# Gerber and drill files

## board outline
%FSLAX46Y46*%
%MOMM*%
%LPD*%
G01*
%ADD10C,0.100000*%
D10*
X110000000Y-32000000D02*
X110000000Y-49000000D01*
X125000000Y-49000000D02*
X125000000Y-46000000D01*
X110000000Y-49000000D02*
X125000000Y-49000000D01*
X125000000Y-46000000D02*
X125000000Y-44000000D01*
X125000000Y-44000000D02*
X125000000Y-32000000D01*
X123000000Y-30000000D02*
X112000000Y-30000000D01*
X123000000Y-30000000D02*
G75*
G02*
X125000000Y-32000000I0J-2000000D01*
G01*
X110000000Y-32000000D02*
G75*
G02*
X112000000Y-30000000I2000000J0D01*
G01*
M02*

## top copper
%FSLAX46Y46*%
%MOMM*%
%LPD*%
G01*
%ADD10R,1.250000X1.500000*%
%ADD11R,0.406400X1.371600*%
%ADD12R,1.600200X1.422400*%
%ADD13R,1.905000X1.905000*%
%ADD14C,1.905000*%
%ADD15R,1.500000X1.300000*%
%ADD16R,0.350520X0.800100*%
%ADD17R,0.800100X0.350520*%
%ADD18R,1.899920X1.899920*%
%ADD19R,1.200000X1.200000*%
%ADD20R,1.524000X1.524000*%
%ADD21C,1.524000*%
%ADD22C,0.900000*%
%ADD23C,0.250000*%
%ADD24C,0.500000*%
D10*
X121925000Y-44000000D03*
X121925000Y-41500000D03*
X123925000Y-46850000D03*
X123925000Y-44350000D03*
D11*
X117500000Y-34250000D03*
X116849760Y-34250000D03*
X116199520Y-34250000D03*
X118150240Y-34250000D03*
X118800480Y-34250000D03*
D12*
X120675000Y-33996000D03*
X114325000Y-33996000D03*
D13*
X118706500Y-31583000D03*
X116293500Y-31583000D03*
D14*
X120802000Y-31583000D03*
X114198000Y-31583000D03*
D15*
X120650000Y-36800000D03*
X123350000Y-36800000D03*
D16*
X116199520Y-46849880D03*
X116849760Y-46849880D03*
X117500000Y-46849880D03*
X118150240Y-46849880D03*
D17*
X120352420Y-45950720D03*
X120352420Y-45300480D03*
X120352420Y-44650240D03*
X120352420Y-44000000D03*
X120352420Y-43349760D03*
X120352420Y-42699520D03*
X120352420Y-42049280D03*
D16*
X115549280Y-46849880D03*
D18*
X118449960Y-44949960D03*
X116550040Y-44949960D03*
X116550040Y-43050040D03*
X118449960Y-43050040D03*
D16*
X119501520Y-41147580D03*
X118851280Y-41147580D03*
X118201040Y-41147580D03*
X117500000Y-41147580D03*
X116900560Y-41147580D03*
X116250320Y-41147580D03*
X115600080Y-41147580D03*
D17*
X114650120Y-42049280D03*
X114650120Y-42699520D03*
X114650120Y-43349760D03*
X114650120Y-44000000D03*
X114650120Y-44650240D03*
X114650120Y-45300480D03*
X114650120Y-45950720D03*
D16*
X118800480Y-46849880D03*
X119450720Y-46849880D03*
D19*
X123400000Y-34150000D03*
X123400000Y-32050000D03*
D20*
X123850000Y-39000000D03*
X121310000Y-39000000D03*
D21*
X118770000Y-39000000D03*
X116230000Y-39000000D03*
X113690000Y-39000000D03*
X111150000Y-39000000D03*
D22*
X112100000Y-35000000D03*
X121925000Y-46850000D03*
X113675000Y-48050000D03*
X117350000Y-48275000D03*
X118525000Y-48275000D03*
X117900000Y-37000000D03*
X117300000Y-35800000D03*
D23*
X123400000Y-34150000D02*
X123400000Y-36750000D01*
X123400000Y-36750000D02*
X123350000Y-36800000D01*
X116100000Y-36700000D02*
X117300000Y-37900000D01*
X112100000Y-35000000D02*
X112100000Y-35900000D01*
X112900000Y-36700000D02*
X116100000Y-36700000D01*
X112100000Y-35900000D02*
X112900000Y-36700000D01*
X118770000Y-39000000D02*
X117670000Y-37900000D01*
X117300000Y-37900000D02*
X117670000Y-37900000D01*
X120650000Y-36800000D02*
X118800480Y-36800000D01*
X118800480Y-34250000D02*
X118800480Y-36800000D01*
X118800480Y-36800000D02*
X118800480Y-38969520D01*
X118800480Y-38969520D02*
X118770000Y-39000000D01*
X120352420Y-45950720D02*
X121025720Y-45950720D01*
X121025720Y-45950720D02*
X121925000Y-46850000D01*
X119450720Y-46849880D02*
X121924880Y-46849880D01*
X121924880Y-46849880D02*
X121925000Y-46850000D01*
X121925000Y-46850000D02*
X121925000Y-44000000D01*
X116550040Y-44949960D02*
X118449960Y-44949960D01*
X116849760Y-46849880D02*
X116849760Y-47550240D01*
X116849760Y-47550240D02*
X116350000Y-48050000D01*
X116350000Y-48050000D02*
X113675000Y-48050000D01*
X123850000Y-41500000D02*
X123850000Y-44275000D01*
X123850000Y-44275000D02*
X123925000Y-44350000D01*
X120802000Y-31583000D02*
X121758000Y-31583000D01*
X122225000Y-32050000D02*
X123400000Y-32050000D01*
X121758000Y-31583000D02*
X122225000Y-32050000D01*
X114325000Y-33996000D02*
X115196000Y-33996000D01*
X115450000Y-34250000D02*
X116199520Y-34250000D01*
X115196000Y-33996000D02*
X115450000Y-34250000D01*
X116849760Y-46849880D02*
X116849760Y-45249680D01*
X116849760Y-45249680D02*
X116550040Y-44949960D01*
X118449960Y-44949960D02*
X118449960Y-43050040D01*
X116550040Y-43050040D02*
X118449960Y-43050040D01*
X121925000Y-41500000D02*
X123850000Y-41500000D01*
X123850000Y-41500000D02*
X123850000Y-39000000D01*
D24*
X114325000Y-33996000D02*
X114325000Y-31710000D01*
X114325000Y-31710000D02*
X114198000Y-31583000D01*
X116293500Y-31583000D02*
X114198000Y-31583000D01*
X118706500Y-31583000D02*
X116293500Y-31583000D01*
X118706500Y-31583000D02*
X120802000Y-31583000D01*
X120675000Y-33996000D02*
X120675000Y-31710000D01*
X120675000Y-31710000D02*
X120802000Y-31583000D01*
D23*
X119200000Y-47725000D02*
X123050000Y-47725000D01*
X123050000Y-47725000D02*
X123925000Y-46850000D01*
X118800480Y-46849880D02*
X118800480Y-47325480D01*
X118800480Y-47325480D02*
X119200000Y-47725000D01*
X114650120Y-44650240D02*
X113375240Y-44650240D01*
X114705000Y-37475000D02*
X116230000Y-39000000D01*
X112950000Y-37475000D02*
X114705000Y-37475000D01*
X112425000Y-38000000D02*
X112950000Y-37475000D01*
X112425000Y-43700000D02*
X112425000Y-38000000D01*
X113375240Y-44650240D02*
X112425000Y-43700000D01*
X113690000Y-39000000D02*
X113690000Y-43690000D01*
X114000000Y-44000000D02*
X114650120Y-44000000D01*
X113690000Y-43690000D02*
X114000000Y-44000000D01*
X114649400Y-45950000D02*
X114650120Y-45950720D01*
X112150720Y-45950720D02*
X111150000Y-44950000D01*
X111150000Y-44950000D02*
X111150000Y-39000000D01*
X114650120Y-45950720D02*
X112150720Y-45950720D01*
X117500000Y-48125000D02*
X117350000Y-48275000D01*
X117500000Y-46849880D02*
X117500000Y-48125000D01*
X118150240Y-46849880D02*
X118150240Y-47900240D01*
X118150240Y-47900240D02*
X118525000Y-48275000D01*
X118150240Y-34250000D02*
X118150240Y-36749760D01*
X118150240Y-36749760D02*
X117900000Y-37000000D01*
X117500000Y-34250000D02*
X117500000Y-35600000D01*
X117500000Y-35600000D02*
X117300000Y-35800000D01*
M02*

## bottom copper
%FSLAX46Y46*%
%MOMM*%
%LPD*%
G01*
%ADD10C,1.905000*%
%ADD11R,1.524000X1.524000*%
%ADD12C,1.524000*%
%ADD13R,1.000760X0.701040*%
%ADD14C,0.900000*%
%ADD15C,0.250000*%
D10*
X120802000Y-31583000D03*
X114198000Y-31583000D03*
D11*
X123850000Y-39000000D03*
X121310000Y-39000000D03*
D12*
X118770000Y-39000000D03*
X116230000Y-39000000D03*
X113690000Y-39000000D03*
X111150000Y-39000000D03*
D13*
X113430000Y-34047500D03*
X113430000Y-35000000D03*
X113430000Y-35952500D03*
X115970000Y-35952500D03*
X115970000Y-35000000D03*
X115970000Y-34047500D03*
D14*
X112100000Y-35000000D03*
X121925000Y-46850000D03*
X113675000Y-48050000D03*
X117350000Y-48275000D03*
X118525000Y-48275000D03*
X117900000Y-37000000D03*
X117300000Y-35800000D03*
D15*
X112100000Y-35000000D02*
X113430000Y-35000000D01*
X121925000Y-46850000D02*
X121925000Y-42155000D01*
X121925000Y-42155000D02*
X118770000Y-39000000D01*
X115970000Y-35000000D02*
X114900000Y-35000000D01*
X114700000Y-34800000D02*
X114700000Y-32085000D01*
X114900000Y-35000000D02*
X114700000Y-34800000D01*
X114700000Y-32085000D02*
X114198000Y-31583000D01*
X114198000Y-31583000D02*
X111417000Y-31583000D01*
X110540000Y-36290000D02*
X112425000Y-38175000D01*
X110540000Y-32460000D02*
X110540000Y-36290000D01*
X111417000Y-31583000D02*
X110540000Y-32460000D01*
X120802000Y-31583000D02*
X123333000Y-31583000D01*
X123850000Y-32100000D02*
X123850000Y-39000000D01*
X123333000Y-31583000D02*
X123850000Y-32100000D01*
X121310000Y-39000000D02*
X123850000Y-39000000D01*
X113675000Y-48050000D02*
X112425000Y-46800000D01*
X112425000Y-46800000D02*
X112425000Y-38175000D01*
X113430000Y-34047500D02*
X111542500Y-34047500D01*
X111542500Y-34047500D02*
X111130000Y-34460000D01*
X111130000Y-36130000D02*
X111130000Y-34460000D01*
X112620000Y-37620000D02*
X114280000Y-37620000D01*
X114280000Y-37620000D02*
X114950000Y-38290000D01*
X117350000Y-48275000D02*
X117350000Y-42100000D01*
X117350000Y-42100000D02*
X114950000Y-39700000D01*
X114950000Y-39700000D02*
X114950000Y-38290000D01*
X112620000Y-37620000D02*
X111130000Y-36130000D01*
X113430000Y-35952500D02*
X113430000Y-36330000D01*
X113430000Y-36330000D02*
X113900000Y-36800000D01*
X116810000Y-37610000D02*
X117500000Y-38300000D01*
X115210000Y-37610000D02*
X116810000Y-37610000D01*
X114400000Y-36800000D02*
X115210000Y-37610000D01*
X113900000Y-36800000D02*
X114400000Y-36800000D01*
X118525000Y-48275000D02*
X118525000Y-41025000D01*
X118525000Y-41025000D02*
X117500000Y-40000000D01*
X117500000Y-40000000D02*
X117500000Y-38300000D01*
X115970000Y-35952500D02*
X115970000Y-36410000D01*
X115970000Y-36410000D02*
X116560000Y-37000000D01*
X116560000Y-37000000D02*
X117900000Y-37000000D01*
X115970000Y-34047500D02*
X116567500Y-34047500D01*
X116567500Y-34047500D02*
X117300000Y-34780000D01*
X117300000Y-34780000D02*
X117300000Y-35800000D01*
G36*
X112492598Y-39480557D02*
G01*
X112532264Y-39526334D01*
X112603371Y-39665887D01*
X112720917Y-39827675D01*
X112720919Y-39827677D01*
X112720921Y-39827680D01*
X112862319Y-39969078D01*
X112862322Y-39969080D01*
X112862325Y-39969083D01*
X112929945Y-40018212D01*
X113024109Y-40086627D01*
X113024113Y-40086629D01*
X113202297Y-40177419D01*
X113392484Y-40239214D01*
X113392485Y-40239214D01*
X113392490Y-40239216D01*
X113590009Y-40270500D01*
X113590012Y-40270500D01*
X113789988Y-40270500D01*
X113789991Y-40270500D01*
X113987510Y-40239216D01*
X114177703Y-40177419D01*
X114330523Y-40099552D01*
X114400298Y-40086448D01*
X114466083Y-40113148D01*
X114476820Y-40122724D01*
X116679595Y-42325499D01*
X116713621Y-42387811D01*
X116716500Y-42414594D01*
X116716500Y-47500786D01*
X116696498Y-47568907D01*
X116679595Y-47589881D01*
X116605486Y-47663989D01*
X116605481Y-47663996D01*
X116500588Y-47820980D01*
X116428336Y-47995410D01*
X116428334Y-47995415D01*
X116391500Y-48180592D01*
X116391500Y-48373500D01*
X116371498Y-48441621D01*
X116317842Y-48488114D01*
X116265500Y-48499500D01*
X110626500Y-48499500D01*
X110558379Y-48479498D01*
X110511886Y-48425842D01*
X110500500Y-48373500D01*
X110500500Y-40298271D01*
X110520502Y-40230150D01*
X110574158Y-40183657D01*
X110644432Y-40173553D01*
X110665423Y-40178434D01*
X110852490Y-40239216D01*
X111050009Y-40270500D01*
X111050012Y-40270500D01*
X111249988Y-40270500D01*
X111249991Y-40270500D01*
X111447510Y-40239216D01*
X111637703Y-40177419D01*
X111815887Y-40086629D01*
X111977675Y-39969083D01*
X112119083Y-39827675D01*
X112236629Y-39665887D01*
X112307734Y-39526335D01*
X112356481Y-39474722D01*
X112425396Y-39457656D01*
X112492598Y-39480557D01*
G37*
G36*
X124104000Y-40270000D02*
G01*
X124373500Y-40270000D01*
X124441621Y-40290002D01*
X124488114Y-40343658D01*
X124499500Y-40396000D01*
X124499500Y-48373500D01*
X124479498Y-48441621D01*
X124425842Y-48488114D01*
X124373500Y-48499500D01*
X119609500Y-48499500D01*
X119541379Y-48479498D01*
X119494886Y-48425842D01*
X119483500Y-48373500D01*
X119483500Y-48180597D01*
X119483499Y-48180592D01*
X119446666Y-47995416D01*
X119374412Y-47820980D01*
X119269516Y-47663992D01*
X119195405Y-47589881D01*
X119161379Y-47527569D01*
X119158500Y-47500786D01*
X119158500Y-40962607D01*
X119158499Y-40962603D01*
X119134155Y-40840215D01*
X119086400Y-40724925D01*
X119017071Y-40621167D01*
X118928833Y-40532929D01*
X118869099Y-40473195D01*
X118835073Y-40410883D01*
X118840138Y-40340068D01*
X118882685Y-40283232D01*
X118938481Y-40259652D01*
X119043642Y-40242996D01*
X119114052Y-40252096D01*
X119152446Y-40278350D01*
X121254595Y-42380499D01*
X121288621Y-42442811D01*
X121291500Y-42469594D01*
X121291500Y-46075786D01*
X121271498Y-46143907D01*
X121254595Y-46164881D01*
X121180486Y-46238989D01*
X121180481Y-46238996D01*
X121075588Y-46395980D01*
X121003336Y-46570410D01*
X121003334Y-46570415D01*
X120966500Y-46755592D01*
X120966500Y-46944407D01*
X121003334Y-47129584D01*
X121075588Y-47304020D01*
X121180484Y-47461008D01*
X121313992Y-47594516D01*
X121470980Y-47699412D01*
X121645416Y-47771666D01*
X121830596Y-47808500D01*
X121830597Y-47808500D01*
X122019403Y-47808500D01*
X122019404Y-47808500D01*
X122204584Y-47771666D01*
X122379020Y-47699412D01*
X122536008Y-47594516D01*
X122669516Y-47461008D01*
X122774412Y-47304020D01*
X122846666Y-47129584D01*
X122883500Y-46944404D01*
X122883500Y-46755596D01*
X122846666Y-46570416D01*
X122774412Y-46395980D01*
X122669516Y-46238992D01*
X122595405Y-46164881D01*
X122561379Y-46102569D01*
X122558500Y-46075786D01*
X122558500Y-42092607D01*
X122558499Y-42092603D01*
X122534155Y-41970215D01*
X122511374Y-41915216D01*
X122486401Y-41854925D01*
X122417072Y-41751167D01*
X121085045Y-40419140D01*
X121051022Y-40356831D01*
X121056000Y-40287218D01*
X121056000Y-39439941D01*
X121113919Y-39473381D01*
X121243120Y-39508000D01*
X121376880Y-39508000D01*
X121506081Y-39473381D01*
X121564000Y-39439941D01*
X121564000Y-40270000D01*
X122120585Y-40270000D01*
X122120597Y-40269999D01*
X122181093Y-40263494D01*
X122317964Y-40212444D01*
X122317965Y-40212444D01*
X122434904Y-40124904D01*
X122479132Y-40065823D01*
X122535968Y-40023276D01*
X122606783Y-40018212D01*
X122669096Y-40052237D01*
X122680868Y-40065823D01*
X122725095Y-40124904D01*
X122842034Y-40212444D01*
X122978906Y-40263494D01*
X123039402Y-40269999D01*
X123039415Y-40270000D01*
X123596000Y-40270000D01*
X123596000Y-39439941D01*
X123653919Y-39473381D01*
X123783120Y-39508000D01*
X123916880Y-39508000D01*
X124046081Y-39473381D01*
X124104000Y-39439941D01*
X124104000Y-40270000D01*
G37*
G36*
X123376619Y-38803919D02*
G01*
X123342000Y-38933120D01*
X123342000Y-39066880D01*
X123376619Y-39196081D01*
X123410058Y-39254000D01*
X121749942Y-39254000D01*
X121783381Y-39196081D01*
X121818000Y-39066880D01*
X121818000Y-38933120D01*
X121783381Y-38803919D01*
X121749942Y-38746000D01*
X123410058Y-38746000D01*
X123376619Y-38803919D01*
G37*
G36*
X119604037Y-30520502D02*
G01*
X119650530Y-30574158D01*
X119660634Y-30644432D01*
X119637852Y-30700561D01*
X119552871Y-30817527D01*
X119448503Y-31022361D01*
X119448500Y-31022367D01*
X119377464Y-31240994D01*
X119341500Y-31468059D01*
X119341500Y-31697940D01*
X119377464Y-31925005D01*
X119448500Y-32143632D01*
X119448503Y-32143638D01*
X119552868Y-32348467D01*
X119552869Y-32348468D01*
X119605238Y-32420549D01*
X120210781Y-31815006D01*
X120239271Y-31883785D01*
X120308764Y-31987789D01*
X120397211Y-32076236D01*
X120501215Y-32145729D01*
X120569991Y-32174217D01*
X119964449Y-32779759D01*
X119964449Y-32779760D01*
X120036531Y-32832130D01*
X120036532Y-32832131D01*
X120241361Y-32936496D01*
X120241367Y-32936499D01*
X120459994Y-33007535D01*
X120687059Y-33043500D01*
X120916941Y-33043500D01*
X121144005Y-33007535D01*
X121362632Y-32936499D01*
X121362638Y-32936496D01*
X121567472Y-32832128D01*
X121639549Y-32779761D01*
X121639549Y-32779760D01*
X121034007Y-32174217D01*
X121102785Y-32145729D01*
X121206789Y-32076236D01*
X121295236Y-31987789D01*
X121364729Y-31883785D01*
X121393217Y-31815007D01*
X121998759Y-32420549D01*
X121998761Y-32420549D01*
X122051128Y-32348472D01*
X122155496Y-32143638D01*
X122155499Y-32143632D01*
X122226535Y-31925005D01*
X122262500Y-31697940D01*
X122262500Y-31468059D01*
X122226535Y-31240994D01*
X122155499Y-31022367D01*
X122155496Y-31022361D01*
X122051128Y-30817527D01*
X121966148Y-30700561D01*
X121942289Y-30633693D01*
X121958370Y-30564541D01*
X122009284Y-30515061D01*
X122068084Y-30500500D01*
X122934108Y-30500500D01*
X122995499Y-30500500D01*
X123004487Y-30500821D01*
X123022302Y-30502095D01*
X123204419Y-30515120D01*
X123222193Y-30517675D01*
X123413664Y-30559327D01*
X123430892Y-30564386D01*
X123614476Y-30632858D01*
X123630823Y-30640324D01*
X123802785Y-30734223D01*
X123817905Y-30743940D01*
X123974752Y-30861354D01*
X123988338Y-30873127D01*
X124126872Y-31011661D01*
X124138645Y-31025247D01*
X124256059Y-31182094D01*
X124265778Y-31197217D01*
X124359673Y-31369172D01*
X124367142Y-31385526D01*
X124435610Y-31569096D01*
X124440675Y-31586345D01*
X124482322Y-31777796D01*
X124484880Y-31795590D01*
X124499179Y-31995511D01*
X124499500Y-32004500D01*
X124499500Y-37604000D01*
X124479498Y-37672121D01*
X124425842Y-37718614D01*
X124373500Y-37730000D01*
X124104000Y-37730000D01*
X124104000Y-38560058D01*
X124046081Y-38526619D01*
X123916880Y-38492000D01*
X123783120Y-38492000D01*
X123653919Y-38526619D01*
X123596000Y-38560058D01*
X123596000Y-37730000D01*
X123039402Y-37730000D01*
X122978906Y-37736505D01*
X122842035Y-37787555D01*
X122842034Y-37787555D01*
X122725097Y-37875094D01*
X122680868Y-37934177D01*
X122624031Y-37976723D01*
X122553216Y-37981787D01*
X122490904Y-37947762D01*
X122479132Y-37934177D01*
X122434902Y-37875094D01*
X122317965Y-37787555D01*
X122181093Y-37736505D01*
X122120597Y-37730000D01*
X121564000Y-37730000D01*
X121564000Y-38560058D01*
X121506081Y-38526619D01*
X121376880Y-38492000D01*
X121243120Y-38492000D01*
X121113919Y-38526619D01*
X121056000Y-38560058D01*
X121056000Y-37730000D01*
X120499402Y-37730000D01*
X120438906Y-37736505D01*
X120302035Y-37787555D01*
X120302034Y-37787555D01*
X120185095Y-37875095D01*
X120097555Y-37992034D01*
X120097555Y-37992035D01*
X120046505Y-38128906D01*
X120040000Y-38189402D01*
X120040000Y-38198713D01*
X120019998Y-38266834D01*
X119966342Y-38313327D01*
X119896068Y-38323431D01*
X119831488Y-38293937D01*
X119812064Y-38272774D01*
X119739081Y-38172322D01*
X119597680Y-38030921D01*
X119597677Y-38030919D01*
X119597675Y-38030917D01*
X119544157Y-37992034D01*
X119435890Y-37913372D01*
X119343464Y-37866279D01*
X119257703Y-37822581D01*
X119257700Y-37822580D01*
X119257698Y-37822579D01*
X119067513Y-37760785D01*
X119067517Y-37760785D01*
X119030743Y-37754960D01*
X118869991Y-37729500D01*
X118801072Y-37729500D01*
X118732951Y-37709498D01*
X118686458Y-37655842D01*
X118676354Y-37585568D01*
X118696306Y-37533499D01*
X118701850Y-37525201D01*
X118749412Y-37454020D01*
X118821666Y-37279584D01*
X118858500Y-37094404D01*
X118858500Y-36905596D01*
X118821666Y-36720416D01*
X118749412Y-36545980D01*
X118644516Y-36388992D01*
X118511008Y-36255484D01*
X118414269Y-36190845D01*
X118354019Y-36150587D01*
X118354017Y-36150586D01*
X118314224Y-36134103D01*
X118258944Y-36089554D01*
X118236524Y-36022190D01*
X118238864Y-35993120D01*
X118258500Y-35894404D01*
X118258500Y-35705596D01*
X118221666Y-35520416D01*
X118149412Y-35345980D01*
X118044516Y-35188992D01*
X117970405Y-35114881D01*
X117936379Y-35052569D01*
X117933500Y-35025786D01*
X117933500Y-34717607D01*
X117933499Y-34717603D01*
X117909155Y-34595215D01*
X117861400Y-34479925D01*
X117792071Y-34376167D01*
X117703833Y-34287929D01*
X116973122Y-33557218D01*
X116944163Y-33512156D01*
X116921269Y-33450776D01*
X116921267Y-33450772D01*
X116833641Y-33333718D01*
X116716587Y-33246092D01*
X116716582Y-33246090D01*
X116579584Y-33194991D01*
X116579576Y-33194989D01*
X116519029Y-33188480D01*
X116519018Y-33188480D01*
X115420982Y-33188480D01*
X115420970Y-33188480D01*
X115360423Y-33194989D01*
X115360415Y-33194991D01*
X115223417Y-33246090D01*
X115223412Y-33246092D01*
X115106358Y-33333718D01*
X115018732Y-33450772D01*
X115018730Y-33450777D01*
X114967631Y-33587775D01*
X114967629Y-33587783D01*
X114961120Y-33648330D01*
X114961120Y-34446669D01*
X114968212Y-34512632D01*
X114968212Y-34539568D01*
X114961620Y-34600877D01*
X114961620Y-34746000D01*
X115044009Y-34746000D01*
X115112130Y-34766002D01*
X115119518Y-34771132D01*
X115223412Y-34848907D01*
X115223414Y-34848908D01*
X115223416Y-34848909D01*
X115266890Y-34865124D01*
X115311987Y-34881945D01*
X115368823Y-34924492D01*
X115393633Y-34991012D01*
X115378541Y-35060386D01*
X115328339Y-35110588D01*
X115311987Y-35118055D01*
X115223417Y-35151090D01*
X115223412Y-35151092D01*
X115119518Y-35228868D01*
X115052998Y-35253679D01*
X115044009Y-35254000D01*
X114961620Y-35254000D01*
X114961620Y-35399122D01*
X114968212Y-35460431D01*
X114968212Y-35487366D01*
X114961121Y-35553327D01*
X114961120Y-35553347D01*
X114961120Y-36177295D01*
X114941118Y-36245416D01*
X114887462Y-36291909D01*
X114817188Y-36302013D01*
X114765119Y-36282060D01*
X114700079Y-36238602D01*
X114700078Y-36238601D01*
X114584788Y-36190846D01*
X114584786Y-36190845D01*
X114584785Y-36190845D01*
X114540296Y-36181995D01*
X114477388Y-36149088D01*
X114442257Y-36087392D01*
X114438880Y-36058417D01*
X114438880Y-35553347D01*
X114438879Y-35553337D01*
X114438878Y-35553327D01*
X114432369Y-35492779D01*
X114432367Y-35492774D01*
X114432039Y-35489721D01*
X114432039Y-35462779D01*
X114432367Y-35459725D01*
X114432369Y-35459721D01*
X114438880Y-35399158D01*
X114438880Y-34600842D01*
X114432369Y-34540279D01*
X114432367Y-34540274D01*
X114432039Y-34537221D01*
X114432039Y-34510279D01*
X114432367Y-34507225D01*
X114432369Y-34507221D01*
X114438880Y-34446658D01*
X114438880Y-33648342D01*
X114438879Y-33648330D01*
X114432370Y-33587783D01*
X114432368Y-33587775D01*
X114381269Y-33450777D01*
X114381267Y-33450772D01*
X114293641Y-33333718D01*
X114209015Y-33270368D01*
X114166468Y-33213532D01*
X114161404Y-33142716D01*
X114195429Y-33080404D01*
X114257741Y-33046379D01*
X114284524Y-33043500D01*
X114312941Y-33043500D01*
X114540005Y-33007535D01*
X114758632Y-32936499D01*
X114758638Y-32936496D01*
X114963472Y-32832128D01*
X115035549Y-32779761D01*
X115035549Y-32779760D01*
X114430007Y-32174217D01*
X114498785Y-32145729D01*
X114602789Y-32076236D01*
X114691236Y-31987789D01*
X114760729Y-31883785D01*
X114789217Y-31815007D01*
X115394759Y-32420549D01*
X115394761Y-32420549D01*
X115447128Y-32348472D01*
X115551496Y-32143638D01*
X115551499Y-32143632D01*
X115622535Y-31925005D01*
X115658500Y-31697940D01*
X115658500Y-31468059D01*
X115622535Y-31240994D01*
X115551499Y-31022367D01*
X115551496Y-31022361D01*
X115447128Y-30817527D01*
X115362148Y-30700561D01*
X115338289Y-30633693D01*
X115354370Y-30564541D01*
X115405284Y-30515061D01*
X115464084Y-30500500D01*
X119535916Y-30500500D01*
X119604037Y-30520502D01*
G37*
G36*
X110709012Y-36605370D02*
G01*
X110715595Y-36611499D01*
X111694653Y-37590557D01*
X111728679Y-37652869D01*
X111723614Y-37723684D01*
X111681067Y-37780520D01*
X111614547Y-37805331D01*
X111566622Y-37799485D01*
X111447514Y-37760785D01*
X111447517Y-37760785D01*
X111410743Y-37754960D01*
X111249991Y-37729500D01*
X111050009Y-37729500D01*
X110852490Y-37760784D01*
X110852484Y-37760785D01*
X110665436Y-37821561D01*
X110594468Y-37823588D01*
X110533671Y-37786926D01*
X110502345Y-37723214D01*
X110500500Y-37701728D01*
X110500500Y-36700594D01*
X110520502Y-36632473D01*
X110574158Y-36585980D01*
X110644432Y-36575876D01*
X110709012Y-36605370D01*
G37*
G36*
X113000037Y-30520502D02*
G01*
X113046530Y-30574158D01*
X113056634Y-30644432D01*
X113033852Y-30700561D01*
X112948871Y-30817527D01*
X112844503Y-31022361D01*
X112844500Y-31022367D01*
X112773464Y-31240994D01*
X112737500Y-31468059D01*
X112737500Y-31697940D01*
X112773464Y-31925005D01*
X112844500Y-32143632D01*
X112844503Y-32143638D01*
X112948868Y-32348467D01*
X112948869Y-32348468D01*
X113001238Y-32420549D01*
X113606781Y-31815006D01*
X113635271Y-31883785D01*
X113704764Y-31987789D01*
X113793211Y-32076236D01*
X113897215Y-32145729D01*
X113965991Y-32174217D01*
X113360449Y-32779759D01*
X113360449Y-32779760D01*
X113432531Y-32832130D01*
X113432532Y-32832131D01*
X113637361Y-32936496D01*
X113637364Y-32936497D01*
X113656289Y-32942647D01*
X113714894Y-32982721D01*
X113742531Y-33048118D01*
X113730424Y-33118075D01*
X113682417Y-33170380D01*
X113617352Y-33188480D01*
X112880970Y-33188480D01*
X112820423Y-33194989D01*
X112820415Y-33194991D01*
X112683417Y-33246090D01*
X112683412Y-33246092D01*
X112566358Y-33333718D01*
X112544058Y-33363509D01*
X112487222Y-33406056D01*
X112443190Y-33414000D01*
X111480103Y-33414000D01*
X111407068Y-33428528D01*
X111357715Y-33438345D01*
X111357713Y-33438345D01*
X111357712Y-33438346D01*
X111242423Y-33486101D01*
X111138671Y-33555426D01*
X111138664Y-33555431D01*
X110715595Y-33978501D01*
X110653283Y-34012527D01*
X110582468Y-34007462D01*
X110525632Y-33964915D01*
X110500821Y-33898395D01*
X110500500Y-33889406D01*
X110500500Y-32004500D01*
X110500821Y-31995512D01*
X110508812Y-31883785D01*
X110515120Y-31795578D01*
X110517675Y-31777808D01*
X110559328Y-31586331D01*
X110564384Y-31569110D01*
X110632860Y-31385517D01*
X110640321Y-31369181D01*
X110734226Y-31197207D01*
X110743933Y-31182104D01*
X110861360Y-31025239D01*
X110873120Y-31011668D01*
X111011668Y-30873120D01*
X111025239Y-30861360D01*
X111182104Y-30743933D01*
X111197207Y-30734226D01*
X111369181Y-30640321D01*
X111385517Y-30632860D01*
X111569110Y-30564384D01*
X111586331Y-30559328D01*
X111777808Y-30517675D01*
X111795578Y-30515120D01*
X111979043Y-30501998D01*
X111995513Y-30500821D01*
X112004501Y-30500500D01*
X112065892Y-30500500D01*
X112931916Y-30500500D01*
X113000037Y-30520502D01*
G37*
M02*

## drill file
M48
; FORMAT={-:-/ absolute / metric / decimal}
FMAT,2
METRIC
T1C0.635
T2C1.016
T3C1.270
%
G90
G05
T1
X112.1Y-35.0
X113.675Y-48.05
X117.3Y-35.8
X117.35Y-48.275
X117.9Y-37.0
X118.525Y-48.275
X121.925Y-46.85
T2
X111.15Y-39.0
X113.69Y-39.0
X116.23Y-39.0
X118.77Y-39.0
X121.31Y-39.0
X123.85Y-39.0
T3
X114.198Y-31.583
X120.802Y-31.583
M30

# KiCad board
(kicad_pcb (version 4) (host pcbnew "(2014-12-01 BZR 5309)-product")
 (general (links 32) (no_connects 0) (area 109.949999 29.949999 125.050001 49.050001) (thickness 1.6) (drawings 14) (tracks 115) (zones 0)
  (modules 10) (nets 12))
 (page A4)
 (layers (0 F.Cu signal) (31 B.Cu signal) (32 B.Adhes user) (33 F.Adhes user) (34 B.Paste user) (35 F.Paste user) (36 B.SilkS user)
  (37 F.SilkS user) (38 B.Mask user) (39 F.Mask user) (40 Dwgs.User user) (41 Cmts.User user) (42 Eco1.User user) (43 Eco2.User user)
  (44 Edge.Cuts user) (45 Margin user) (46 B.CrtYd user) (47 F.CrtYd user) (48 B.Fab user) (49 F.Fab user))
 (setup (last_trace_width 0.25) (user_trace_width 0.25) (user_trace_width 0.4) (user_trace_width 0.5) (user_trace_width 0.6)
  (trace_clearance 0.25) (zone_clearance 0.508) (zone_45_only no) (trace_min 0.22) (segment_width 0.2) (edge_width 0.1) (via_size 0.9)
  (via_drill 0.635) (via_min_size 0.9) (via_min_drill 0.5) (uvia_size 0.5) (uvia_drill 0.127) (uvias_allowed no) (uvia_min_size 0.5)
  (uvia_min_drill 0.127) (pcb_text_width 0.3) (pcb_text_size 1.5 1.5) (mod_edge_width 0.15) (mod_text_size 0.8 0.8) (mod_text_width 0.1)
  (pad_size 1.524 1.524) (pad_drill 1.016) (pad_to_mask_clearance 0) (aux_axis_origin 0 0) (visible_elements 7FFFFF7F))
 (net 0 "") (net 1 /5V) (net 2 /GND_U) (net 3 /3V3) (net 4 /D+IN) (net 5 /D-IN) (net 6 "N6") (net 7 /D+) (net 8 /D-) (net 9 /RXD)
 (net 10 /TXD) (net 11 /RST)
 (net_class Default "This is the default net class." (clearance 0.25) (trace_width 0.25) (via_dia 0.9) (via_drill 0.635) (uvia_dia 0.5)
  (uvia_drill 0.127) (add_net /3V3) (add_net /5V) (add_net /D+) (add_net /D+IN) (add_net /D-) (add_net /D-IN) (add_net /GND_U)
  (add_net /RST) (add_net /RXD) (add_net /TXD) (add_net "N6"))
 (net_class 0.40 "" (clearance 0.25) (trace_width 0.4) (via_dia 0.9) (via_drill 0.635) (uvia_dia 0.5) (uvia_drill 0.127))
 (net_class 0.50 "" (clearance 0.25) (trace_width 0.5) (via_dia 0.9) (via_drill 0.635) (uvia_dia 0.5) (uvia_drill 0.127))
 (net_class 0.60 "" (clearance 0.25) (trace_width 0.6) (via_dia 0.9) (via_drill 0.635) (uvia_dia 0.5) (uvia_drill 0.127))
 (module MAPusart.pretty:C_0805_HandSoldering (layer F.Cu) (at 121.925 42.75 90)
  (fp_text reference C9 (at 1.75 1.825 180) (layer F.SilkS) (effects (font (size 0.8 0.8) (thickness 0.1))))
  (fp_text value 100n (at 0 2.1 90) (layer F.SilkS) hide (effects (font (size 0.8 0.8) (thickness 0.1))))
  (pad 1 smd rect (at -1.25 0 90) (size 1.5 1.25) (layers F.Cu F.Paste F.Mask) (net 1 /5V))
  (pad 2 smd rect (at 1.25 0 90) (size 1.5 1.25) (layers F.Cu F.Paste F.Mask) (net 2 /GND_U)))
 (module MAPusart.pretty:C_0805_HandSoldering (layer F.Cu) (at 123.925 45.6 90)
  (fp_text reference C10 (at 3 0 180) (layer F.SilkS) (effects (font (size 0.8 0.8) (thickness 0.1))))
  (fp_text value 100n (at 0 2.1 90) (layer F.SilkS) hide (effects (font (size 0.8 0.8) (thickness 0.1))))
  (pad 1 smd rect (at -1.25 0 90) (size 1.5 1.25) (layers F.Cu F.Paste F.Mask) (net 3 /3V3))
  (pad 2 smd rect (at 1.25 0 90) (size 1.5 1.25) (layers F.Cu F.Paste F.Mask) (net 2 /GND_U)))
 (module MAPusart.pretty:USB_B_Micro (layer F.Cu) (at 117.5 34.25 270)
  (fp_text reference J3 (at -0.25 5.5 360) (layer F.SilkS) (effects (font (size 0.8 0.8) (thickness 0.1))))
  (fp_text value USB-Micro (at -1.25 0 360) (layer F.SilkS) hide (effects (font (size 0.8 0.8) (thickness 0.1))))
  (pad 3 smd rect (at 0 0 270) (size 1.3716 0.4064) (layers F.Cu F.Paste F.Mask) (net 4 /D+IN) (clearance 0.2032))
  (pad 4 smd rect (at 0 0.65024 270) (size 1.3716 0.4064) (layers F.Cu F.Paste F.Mask) (clearance 0.2032))
  (pad 5 smd rect (at 0 1.30048 270) (size 1.3716 0.4064) (layers F.Cu F.Paste F.Mask) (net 2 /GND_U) (clearance 0.2032))
  (pad 2 smd rect (at 0 -0.65024 270) (size 1.3716 0.4064) (layers F.Cu F.Paste F.Mask) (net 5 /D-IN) (clearance 0.2032))
  (pad 1 smd rect (at 0 -1.30048 270) (size 1.3716 0.4064) (layers F.Cu F.Paste F.Mask) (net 1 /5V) (clearance 0.2032))
  (pad T1 smd rect (at -0.254 -3.175 270) (size 1.4224 1.6002) (layers F.Cu F.Paste F.Mask) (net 2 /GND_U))
  (pad T2 smd rect (at -0.254 3.175 270) (size 1.4224 1.6002) (layers F.Cu F.Paste F.Mask) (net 2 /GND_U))
  (pad T3 smd rect (at -2.667 -1.2065 270) (size 1.905 1.905) (layers F.Cu F.Paste F.Mask) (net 2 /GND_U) (clearance 0.2032))
  (pad T4 smd rect (at -2.667 1.2065 270) (size 1.905 1.905) (layers F.Cu F.Paste F.Mask) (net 2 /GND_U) (clearance 0.2032))
  (pad T5 thru_hole circle (at -2.667 -3.302 270) (size 1.905 1.905) (drill 1.27) (layers *.Cu *.Paste *.Mask F.SilkS) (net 2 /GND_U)
   (clearance 0.2032))
  (pad T6 thru_hole circle (at -2.667 3.302 270) (size 1.905 1.905) (drill 1.27) (layers *.Cu *.Paste *.Mask F.SilkS) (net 2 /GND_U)
   (clearance 0.2032)))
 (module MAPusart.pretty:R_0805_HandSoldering (layer F.Cu) (at 122 36.8)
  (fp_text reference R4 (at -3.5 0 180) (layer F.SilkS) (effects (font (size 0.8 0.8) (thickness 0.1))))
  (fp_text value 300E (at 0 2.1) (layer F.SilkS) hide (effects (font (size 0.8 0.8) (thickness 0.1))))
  (pad 1 smd rect (at -1.35 0) (size 1.5 1.3) (layers F.Cu F.Paste F.Mask) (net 1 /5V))
  (pad 2 smd rect (at 1.35 0) (size 1.5 1.3) (layers F.Cu F.Paste F.Mask) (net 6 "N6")))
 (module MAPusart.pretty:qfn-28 (layer F.Cu) (at 117.5 44)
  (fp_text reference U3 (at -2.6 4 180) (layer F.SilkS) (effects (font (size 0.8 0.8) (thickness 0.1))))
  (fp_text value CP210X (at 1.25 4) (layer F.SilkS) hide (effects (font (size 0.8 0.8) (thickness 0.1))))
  (pad 2 smd rect (at -1.30048 2.84988) (size 0.35052 0.8001) (layers F.Cu F.Paste F.Mask) (solder_mask_margin 0.07112) (clearance 0.1))
  (pad 3 smd rect (at -0.65024 2.84988) (size 0.35052 0.8001) (layers F.Cu F.Paste F.Mask) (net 2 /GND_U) (solder_mask_margin 0.07112)
   (clearance 0.1))
  (pad 4 smd rect (at 0 2.84988) (size 0.35052 0.8001) (layers F.Cu F.Paste F.Mask) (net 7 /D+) (solder_mask_margin 0.07112) (clearance 0.1))
  (pad 5 smd rect (at 0.65024 2.84988) (size 0.35052 0.8001) (layers F.Cu F.Paste F.Mask) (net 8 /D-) (solder_mask_margin 0.07112)
   (clearance 0.1))
  (pad 8 smd rect (at 2.85242 1.95072) (size 0.8001 0.35052) (layers F.Cu F.Paste F.Mask) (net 1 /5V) (solder_mask_margin 0.07112)
   (clearance 0.1))
  (pad 9 smd rect (at 2.85242 1.30048) (size 0.8001 0.35052) (layers F.Cu F.Paste F.Mask) (solder_mask_margin 0.07112) (clearance 0.1))
  (pad 10 smd rect (at 2.85242 0.65024) (size 0.8001 0.35052) (layers F.Cu F.Paste F.Mask) (solder_mask_margin 0.07112) (clearance 0.1))
  (pad 11 smd rect (at 2.85242 0) (size 0.8001 0.35052) (layers F.Cu F.Paste F.Mask) (solder_mask_margin 0.07112) (clearance 0.1))
  (pad 12 smd rect (at 2.85242 -0.65024) (size 0.8001 0.35052) (layers F.Cu F.Paste F.Mask) (solder_mask_margin 0.07112) (clearance 0.1))
  (pad 13 smd rect (at 2.85242 -1.30048) (size 0.8001 0.35052) (layers F.Cu F.Paste F.Mask) (solder_mask_margin 0.07112) (clearance 0.1))
  (pad 14 smd rect (at 2.85242 -1.95072) (size 0.8001 0.35052) (layers F.Cu F.Paste F.Mask) (solder_mask_margin 0.07112) (clearance 0.1))
  (pad 1 smd rect (at -1.95072 2.84988) (size 0.35052 0.8001) (layers F.Cu F.Paste F.Mask) (solder_mask_margin 0.07112) (clearance 0.1))
  (pad 29 smd rect (at 0.94996 0.94996) (size 1.89992 1.89992) (layers F.Cu F.Paste F.Mask) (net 2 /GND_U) (solder_mask_margin 0.07112)
   (solder_paste_margin -0.09906))
  (pad 29 smd rect (at -0.94996 0.94996) (size 1.89992 1.89992) (layers F.Cu F.Paste F.Mask) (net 2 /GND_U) (solder_mask_margin 0.07112)
   (solder_paste_margin -0.09906))
  (pad 29 smd rect (at -0.94996 -0.94996) (size 1.89992 1.89992) (layers F.Cu F.Paste F.Mask) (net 2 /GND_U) (solder_mask_margin 0.07112)
   (solder_paste_margin -0.09906))
  (pad 29 smd rect (at 0.94996 -0.94996) (size 1.89992 1.89992) (layers F.Cu F.Paste F.Mask) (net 2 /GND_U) (solder_mask_margin 0.07112)
   (solder_paste_margin -0.09906))
  (pad 15 smd rect (at 2.00152 -2.85242) (size 0.35052 0.8001) (layers F.Cu F.Paste F.Mask) (solder_mask_margin 0.07112) (clearance 0.1))
  (pad 16 smd rect (at 1.35128 -2.85242) (size 0.35052 0.8001) (layers F.Cu F.Paste F.Mask) (solder_mask_margin 0.07112) (clearance 0.1))
  (pad 17 smd rect (at 0.70104 -2.85242) (size 0.35052 0.8001) (layers F.Cu F.Paste F.Mask) (solder_mask_margin 0.07112) (clearance 0.1))
  (pad 18 smd rect (at 0 -2.85242) (size 0.35052 0.8001) (layers F.Cu F.Paste F.Mask) (solder_mask_margin 0.07112) (clearance 0.1))
  (pad 19 smd rect (at -0.59944 -2.85242) (size 0.35052 0.8001) (layers F.Cu F.Paste F.Mask) (solder_mask_margin 0.07112) (clearance 0.1))
  (pad 20 smd rect (at -1.24968 -2.85242) (size 0.35052 0.8001) (layers F.Cu F.Paste F.Mask) (solder_mask_margin 0.07112) (clearance 0.1))
  (pad 21 smd rect (at -1.89992 -2.85242) (size 0.35052 0.8001) (layers F.Cu F.Paste F.Mask) (solder_mask_margin 0.07112) (clearance 0.1))
  (pad 22 smd rect (at -2.84988 -1.95072) (size 0.8001 0.35052) (layers F.Cu F.Paste F.Mask) (solder_mask_margin 0.07112) (clearance 0.1))
  (pad 23 smd rect (at -2.84988 -1.30048) (size 0.8001 0.35052) (layers F.Cu F.Paste F.Mask) (solder_mask_margin 0.07112) (clearance 0.1))
  (pad 24 smd rect (at -2.84988 -0.65024) (size 0.8001 0.35052) (layers F.Cu F.Paste F.Mask) (solder_mask_margin 0.07112) (clearance 0.1))
  (pad 25 smd rect (at -2.84988 0) (size 0.8001 0.35052) (layers F.Cu F.Paste F.Mask) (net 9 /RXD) (solder_mask_margin 0.07112)
   (clearance 0.1))
  (pad 26 smd rect (at -2.84988 0.65024) (size 0.8001 0.35052) (layers F.Cu F.Paste F.Mask) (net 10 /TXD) (solder_mask_margin 0.07112)
   (clearance 0.1))
  (pad 27 smd rect (at -2.84988 1.30048) (size 0.8001 0.35052) (layers F.Cu F.Paste F.Mask) (solder_mask_margin 0.07112) (clearance 0.1))
  (pad 28 smd rect (at -2.84988 1.95072) (size 0.8001 0.35052) (layers F.Cu F.Paste F.Mask) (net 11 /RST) (solder_mask_margin 0.07112)
   (clearance 0.1))
  (pad 6 smd rect (at 1.30048 2.84988) (size 0.35052 0.8001) (layers F.Cu F.Paste F.Mask) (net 3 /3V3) (solder_mask_margin 0.07112)
   (clearance 0.1))
  (pad 7 smd rect (at 1.95072 2.84988) (size 0.35052 0.8001) (layers F.Cu F.Paste F.Mask) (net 1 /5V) (solder_mask_margin 0.07112)
   (clearance 0.1)))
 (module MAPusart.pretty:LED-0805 (layer F.Cu) (at 123.4 33.1 90)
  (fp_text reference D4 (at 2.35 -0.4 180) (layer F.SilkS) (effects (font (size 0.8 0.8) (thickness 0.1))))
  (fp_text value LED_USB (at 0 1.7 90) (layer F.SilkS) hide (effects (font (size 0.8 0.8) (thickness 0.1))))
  (pad 1 smd rect (at -1.05 0 90) (size 1.2 1.2) (layers F.Cu F.Paste F.Mask) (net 6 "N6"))
  (pad 2 smd rect (at 1.05 0 90) (size 1.2 1.2) (layers F.Cu F.Paste F.Mask) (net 2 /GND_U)))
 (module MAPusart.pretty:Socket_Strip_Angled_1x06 (layer B.Cu) (at 117.5 39)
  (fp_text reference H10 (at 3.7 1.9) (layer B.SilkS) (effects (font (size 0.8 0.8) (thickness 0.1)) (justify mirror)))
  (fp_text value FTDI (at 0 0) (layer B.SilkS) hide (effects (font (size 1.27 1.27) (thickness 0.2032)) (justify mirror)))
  (pad 1 thru_hole rect (at 6.35 0) (size 1.524 1.524) (drill 1.016) (layers *.Cu *.Mask B.SilkS) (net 2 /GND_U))
  (pad 2 thru_hole rect (at 3.81 0) (size 1.524 1.524) (drill 1.016) (layers *.Cu *.Mask B.SilkS) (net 2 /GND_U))
  (pad 3 thru_hole circle (at 1.27 0) (size 1.524 1.524) (drill 1.016) (layers *.Cu *.Mask B.SilkS) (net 1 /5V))
  (pad 4 thru_hole circle (at -1.27 0) (size 1.524 1.524) (drill 1.016) (layers *.Cu *.Mask B.SilkS) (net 10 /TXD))
  (pad 5 thru_hole circle (at -3.81 0) (size 1.524 1.524) (drill 1.016) (layers *.Cu *.Mask B.SilkS) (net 9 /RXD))
  (pad 6 thru_hole circle (at -6.35 0) (size 1.524 1.524) (drill 1.016) (layers *.Cu *.Mask B.SilkS) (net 11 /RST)))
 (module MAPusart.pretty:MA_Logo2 (layer B.Cu) (at 117.5 44.5 180)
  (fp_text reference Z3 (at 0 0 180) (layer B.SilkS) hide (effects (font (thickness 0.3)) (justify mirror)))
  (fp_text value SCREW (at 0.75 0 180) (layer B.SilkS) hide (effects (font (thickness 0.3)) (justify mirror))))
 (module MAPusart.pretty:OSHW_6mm (layer B.Cu) (at 120.8 33.9 180)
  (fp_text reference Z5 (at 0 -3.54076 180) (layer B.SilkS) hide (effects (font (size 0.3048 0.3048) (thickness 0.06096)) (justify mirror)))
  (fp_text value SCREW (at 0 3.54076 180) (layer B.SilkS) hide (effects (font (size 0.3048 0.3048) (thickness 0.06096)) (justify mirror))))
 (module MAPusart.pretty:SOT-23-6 (layer B.Cu) (at 114.7 35 270)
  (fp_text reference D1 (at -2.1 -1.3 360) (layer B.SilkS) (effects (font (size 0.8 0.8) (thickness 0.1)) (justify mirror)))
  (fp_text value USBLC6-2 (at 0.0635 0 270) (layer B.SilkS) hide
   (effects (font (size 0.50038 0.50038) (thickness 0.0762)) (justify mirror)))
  (pad 6 smd rect (at -0.9525 1.27 270) (size 0.70104 1.00076) (layers B.Cu B.Paste B.Mask) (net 7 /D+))
  (pad 5 smd rect (at 0 1.27 270) (size 0.70104 1.00076) (layers B.Cu B.Paste B.Mask) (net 1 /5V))
  (pad 4 smd rect (at 0.9525 1.27 270) (size 0.70104 1.00076) (layers B.Cu B.Paste B.Mask) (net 8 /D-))
  (pad 3 smd rect (at 0.9525 -1.27 270) (size 0.70104 1.00076) (layers B.Cu B.Paste B.Mask) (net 5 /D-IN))
  (pad 2 smd rect (at 0 -1.27 270) (size 0.70104 1.00076) (layers B.Cu B.Paste B.Mask) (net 2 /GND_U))
  (pad 1 smd rect (at -0.9525 -1.27 270) (size 0.70104 1.00076) (layers B.Cu B.Paste B.Mask) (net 4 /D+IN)))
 (gr_line (start 110 32) (end 110 49) (angle 90) (layer Edge.Cuts) (width 0.1))
 (gr_line (start 125 49) (end 125 46) (angle 90) (layer Edge.Cuts) (width 0.1))
 (gr_line (start 110 49) (end 125 49) (angle 90) (layer Edge.Cuts) (width 0.1))
 (gr_line (start 125 46) (end 125 44) (angle 90) (layer Edge.Cuts) (width 0.1))
 (gr_line (start 125 44) (end 125 32) (angle 90) (layer Edge.Cuts) (width 0.1))
 (gr_line (start 123 30) (end 112 30) (angle 90) (layer Edge.Cuts) (width 0.1))
 (gr_arc (start 123 32) (end 123 30) (angle 90) (layer Edge.Cuts) (width 0.1))
 (gr_arc (start 112 32) (end 110 32) (angle 90) (layer Edge.Cuts) (width 0.1))
 (segment (start 123.4 34.15) (end 123.4 36.75) (width 0.25) (layer F.Cu) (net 6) (status 30))
 (segment (start 123.4 36.75) (end 123.35 36.8) (width 0.25) (layer F.Cu) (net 6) (status 30))
 (segment (start 116.1 36.7) (end 117.3 37.9) (width 0.25) (layer F.Cu) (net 1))
 (segment (start 112.1 35) (end 112.1 35.9) (width 0.25) (layer F.Cu) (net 1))
 (segment (start 112.9 36.7) (end 116.1 36.7) (width 0.25) (layer F.Cu) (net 1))
 (segment (start 112.1 35.9) (end 112.9 36.7) (width 0.25) (layer F.Cu) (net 1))
 (segment (start 118.77 39) (end 117.67 37.9) (width 0.25) (layer F.Cu) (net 1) (status 10))
 (segment (start 117.3 37.9) (end 117.67 37.9) (width 0.25) (layer F.Cu) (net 1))
 (segment (start 112.1 35) (end 113.43 35) (width 0.25) (layer B.Cu) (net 1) (status 20))
 (via (at 112.1 35) (size 0.9) (layers F.Cu B.Cu) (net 1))
 (segment (start 120.65 36.8) (end 118.80048 36.8) (width 0.25) (layer F.Cu) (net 1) (status 10))
 (segment (start 118.80048 34.25) (end 118.80048 36.8) (width 0.25) (layer F.Cu) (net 1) (status 10))
 (segment (start 118.80048 36.8) (end 118.80048 38.96952) (width 0.25) (layer F.Cu) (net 1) (status 20))
 (segment (start 118.80048 38.96952) (end 118.77 39) (width 0.25) (layer F.Cu) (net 1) (status 30))
 (segment (start 121.925 46.85) (end 121.925 42.155) (width 0.25) (layer B.Cu) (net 1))
 (segment (start 121.925 42.155) (end 118.77 39) (width 0.25) (layer B.Cu) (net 1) (status 20))
 (segment (start 120.35242 45.95072) (end 121.02572 45.95072) (width 0.25) (layer F.Cu) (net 1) (status 10))
 (segment (start 121.02572 45.95072) (end 121.925 46.85) (width 0.25) (layer F.Cu) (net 1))
 (segment (start 119.45072 46.84988) (end 121.92488 46.84988) (width 0.25) (layer F.Cu) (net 1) (status 10))
 (segment (start 121.92488 46.84988) (end 121.925 46.85) (width 0.25) (layer F.Cu) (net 1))
 (via (at 121.925 46.85) (size 0.9) (layers F.Cu B.Cu) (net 1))
 (segment (start 121.925 46.85) (end 121.925 44) (width 0.25) (layer F.Cu) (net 1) (status 20))
 (segment (start 115.97 35) (end 114.9 35) (width 0.25) (layer B.Cu) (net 2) (status 10))
 (segment (start 114.7 34.8) (end 114.7 32.085) (width 0.25) (layer B.Cu) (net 2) (status 20))
 (segment (start 114.9 35) (end 114.7 34.8) (width 0.25) (layer B.Cu) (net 2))
 (segment (start 114.7 32.085) (end 114.198 31.583) (width 0.25) (layer B.Cu) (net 2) (status 30))
 (segment (start 114.198 31.583) (end 111.417 31.583) (width 0.25) (layer B.Cu) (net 2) (status 10))
 (segment (start 110.54 36.29) (end 112.425 38.175) (width 0.25) (layer B.Cu) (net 2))
 (segment (start 110.54 32.46) (end 110.54 36.29) (width 0.25) (layer B.Cu) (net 2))
 (segment (start 111.417 31.583) (end 110.54 32.46) (width 0.25) (layer B.Cu) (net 2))
 (segment (start 120.802 31.583) (end 123.333 31.583) (width 0.25) (layer B.Cu) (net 2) (status 10))
 (segment (start 123.85 32.1) (end 123.85 39) (width 0.25) (layer B.Cu) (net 2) (status 20))
 (segment (start 123.333 31.583) (end 123.85 32.1) (width 0.25) (layer B.Cu) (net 2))
 (segment (start 121.31 39) (end 123.85 39) (width 0.25) (layer B.Cu) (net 2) (status 30))
 (segment (start 116.55004 44.94996) (end 118.44996 44.94996) (width 0.25) (layer F.Cu) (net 2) (status 30))
 (segment (start 116.84976 46.84988) (end 116.84976 47.55024) (width 0.25) (layer F.Cu) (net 2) (status 10))
 (segment (start 116.84976 47.55024) (end 116.35 48.05) (width 0.25) (layer F.Cu) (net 2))
 (segment (start 116.35 48.05) (end 113.675 48.05) (width 0.25) (layer F.Cu) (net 2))
 (via (at 113.675 48.05) (size 0.9) (layers F.Cu B.Cu) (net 2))
 (segment (start 113.675 48.05) (end 112.425 46.8) (width 0.25) (layer B.Cu) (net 2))
 (segment (start 112.425 46.8) (end 112.425 38.175) (width 0.25) (layer B.Cu) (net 2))
 (segment (start 123.85 41.5) (end 123.85 44.275) (width 0.25) (layer F.Cu) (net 2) (status 20))
 (segment (start 123.85 44.275) (end 123.925 44.35) (width 0.25) (layer F.Cu) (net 2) (status 30))
 (segment (start 120.802 31.583) (end 121.758 31.583) (width 0.25) (layer F.Cu) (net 2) (status 10))
 (segment (start 122.225 32.05) (end 123.4 32.05) (width 0.25) (layer F.Cu) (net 2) (status 20))
 (segment (start 121.758 31.583) (end 122.225 32.05) (width 0.25) (layer F.Cu) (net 2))
 (segment (start 114.325 33.996) (end 115.196 33.996) (width 0.25) (layer F.Cu) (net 2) (status 10))
 (segment (start 115.45 34.25) (end 116.19952 34.25) (width 0.25) (layer F.Cu) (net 2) (status 20))
 (segment (start 115.196 33.996) (end 115.45 34.25) (width 0.25) (layer F.Cu) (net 2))
 (segment (start 116.84976 46.84988) (end 116.84976 45.24968) (width 0.25) (layer F.Cu) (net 2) (status 30))
 (segment (start 116.84976 45.24968) (end 116.55004 44.94996) (width 0.25) (layer F.Cu) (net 2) (status 30))
 (segment (start 118.44996 44.94996) (end 118.44996 43.05004) (width 0.25) (layer F.Cu) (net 2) (status 30))
 (segment (start 116.55004 43.05004) (end 118.44996 43.05004) (width 0.25) (layer F.Cu) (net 2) (status 30))
 (segment (start 121.925 41.5) (end 123.85 41.5) (width 0.25) (layer F.Cu) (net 2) (status 10))
 (segment (start 123.85 41.5) (end 123.85 39) (width 0.25) (layer F.Cu) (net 2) (status 20))
 (segment (start 114.325 33.996) (end 114.325 31.71) (width 0.5) (layer F.Cu) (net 2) (status 30))
 (segment (start 114.325 31.71) (end 114.198 31.583) (width 0.5) (layer F.Cu) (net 2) (status 30))
 (segment (start 116.2935 31.583) (end 114.198 31.583) (width 0.5) (layer F.Cu) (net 2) (status 30))
 (segment (start 118.7065 31.583) (end 116.2935 31.583) (width 0.5) (layer F.Cu) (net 2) (status 30))
 (segment (start 118.7065 31.583) (end 120.802 31.583) (width 0.5) (layer F.Cu) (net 2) (status 30))
 (segment (start 120.675 33.996) (end 120.675 31.71) (width 0.5) (layer F.Cu) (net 2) (status 30))
 (segment (start 120.675 31.71) (end 120.802 31.583) (width 0.5) (layer F.Cu) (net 2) (status 30))
 (segment (start 119.2 47.725) (end 123.05 47.725) (width 0.25) (layer F.Cu) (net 3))
 (segment (start 123.05 47.725) (end 123.925 46.85) (width 0.25) (layer F.Cu) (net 3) (status 20))
 (segment (start 118.80048 46.84988) (end 118.80048 47.32548) (width 0.25) (layer F.Cu) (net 3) (status 10))
 (segment (start 118.80048 47.32548) (end 119.2 47.725) (width 0.25) (layer F.Cu) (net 3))
 (segment (start 114.65012 44.65024) (end 113.37524 44.65024) (width 0.25) (layer F.Cu) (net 10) (status 10))
 (segment (start 114.705 37.475) (end 116.23 39) (width 0.25) (layer F.Cu) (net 10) (status 20))
 (segment (start 112.95 37.475) (end 114.705 37.475) (width 0.25) (layer F.Cu) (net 10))
 (segment (start 112.425 38) (end 112.95 37.475) (width 0.25) (layer F.Cu) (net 10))
 (segment (start 112.425 43.7) (end 112.425 38) (width 0.25) (layer F.Cu) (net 10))
 (segment (start 113.37524 44.65024) (end 112.425 43.7) (width 0.25) (layer F.Cu) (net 10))
 (segment (start 113.69 39) (end 113.69 43.69) (width 0.25) (layer F.Cu) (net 9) (status 10))
 (segment (start 114 44) (end 114.65012 44) (width 0.25) (layer F.Cu) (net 9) (status 20))
 (segment (start 113.69 43.69) (end 114 44) (width 0.25) (layer F.Cu) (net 9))
 (segment (start 114.6494 45.95) (end 114.65012 45.95072) (width 0.25) (layer F.Cu) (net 11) (status 30))
 (segment (start 112.15072 45.95072) (end 111.15 44.95) (width 0.25) (layer F.Cu) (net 11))
 (segment (start 111.15 44.95) (end 111.15 39) (width 0.25) (layer F.Cu) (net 11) (status 20))
 (segment (start 114.65012 45.95072) (end 112.15072 45.95072) (width 0.25) (layer F.Cu) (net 11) (status 10))
 (segment (start 113.43 34.0475) (end 111.5425 34.0475) (width 0.25) (layer B.Cu) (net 7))
 (segment (start 111.5425 34.0475) (end 111.13 34.46) (width 0.25) (layer B.Cu) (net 7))
 (segment (start 111.13 36.13) (end 111.13 34.46) (width 0.25) (layer B.Cu) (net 7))
 (segment (start 112.62 37.62) (end 114.28 37.62) (width 0.25) (layer B.Cu) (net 7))
 (segment (start 114.28 37.62) (end 114.95 38.29) (width 0.25) (layer B.Cu) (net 7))
 (segment (start 117.5 48.125) (end 117.35 48.275) (width 0.25) (layer F.Cu) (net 7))
 (segment (start 117.35 48.275) (end 117.35 42.1) (width 0.25) (layer B.Cu) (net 7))
 (segment (start 117.35 42.1) (end 114.95 39.7) (width 0.25) (layer B.Cu) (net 7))
 (segment (start 117.5 46.84988) (end 117.5 48.125) (width 0.25) (layer F.Cu) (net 7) (status 10))
 (segment (start 114.95 39.7) (end 114.95 38.29) (width 0.25) (layer B.Cu) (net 7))
 (via (at 117.35 48.275) (size 0.9) (layers F.Cu B.Cu) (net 7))
 (segment (start 112.62 37.62) (end 111.13 36.13) (width 0.25) (layer B.Cu) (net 7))
 (segment (start 113.43 35.9525) (end 113.43 36.33) (width 0.25) (layer B.Cu) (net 8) (status 10))
 (segment (start 113.43 36.33) (end 113.9 36.8) (width 0.25) (layer B.Cu) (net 8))
 (segment (start 116.81 37.61) (end 117.5 38.3) (width 0.25) (layer B.Cu) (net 8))
 (segment (start 115.21 37.61) (end 116.81 37.61) (width 0.25) (layer B.Cu) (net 8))
 (segment (start 114.4 36.8) (end 115.21 37.61) (width 0.25) (layer B.Cu) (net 8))
 (segment (start 113.9 36.8) (end 114.4 36.8) (width 0.25) (layer B.Cu) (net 8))
 (segment (start 118.525 48.275) (end 118.525 41.025) (width 0.25) (layer B.Cu) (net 8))
 (segment (start 118.525 41.025) (end 117.5 40) (width 0.25) (layer B.Cu) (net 8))
 (segment (start 118.15024 46.84988) (end 118.15024 47.90024) (width 0.25) (layer F.Cu) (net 8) (status 10))
 (segment (start 118.15024 47.90024) (end 118.525 48.275) (width 0.25) (layer F.Cu) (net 8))
 (via (at 118.525 48.275) (size 0.9) (layers F.Cu B.Cu) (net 8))
 (segment (start 117.5 40) (end 117.5 38.3) (width 0.25) (layer B.Cu) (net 8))
 (segment (start 115.97 35.9525) (end 115.97 36.41) (width 0.25) (layer B.Cu) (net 5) (status 10))
 (segment (start 115.97 36.41) (end 116.56 37) (width 0.25) (layer B.Cu) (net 5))
 (segment (start 118.15024 34.25) (end 118.15024 36.74976) (width 0.25) (layer F.Cu) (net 5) (status 10))
 (segment (start 118.15024 36.74976) (end 117.9 37) (width 0.25) (layer F.Cu) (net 5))
 (via (at 117.9 37) (size 0.9) (layers F.Cu B.Cu) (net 5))
 (segment (start 116.56 37) (end 117.9 37) (width 0.25) (layer B.Cu) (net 5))
 (segment (start 115.97 34.0475) (end 116.5675 34.0475) (width 0.25) (layer B.Cu) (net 4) (status 10))
 (segment (start 116.5675 34.0475) (end 117.3 34.78) (width 0.25) (layer B.Cu) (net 4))
 (segment (start 117.3 34.78) (end 117.3 35.8) (width 0.25) (layer B.Cu) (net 4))
 (segment (start 117.5 34.25) (end 117.5 35.6) (width 0.25) (layer F.Cu) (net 4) (status 10))
 (via (at 117.3 35.8) (size 0.9) (layers F.Cu B.Cu) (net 4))
 (segment (start 117.5 35.6) (end 117.3 35.8) (width 0.25) (layer F.Cu) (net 4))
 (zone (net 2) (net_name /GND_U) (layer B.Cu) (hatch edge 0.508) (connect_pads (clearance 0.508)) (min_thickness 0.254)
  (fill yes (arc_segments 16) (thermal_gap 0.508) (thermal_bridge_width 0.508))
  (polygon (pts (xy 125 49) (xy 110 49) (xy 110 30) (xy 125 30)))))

